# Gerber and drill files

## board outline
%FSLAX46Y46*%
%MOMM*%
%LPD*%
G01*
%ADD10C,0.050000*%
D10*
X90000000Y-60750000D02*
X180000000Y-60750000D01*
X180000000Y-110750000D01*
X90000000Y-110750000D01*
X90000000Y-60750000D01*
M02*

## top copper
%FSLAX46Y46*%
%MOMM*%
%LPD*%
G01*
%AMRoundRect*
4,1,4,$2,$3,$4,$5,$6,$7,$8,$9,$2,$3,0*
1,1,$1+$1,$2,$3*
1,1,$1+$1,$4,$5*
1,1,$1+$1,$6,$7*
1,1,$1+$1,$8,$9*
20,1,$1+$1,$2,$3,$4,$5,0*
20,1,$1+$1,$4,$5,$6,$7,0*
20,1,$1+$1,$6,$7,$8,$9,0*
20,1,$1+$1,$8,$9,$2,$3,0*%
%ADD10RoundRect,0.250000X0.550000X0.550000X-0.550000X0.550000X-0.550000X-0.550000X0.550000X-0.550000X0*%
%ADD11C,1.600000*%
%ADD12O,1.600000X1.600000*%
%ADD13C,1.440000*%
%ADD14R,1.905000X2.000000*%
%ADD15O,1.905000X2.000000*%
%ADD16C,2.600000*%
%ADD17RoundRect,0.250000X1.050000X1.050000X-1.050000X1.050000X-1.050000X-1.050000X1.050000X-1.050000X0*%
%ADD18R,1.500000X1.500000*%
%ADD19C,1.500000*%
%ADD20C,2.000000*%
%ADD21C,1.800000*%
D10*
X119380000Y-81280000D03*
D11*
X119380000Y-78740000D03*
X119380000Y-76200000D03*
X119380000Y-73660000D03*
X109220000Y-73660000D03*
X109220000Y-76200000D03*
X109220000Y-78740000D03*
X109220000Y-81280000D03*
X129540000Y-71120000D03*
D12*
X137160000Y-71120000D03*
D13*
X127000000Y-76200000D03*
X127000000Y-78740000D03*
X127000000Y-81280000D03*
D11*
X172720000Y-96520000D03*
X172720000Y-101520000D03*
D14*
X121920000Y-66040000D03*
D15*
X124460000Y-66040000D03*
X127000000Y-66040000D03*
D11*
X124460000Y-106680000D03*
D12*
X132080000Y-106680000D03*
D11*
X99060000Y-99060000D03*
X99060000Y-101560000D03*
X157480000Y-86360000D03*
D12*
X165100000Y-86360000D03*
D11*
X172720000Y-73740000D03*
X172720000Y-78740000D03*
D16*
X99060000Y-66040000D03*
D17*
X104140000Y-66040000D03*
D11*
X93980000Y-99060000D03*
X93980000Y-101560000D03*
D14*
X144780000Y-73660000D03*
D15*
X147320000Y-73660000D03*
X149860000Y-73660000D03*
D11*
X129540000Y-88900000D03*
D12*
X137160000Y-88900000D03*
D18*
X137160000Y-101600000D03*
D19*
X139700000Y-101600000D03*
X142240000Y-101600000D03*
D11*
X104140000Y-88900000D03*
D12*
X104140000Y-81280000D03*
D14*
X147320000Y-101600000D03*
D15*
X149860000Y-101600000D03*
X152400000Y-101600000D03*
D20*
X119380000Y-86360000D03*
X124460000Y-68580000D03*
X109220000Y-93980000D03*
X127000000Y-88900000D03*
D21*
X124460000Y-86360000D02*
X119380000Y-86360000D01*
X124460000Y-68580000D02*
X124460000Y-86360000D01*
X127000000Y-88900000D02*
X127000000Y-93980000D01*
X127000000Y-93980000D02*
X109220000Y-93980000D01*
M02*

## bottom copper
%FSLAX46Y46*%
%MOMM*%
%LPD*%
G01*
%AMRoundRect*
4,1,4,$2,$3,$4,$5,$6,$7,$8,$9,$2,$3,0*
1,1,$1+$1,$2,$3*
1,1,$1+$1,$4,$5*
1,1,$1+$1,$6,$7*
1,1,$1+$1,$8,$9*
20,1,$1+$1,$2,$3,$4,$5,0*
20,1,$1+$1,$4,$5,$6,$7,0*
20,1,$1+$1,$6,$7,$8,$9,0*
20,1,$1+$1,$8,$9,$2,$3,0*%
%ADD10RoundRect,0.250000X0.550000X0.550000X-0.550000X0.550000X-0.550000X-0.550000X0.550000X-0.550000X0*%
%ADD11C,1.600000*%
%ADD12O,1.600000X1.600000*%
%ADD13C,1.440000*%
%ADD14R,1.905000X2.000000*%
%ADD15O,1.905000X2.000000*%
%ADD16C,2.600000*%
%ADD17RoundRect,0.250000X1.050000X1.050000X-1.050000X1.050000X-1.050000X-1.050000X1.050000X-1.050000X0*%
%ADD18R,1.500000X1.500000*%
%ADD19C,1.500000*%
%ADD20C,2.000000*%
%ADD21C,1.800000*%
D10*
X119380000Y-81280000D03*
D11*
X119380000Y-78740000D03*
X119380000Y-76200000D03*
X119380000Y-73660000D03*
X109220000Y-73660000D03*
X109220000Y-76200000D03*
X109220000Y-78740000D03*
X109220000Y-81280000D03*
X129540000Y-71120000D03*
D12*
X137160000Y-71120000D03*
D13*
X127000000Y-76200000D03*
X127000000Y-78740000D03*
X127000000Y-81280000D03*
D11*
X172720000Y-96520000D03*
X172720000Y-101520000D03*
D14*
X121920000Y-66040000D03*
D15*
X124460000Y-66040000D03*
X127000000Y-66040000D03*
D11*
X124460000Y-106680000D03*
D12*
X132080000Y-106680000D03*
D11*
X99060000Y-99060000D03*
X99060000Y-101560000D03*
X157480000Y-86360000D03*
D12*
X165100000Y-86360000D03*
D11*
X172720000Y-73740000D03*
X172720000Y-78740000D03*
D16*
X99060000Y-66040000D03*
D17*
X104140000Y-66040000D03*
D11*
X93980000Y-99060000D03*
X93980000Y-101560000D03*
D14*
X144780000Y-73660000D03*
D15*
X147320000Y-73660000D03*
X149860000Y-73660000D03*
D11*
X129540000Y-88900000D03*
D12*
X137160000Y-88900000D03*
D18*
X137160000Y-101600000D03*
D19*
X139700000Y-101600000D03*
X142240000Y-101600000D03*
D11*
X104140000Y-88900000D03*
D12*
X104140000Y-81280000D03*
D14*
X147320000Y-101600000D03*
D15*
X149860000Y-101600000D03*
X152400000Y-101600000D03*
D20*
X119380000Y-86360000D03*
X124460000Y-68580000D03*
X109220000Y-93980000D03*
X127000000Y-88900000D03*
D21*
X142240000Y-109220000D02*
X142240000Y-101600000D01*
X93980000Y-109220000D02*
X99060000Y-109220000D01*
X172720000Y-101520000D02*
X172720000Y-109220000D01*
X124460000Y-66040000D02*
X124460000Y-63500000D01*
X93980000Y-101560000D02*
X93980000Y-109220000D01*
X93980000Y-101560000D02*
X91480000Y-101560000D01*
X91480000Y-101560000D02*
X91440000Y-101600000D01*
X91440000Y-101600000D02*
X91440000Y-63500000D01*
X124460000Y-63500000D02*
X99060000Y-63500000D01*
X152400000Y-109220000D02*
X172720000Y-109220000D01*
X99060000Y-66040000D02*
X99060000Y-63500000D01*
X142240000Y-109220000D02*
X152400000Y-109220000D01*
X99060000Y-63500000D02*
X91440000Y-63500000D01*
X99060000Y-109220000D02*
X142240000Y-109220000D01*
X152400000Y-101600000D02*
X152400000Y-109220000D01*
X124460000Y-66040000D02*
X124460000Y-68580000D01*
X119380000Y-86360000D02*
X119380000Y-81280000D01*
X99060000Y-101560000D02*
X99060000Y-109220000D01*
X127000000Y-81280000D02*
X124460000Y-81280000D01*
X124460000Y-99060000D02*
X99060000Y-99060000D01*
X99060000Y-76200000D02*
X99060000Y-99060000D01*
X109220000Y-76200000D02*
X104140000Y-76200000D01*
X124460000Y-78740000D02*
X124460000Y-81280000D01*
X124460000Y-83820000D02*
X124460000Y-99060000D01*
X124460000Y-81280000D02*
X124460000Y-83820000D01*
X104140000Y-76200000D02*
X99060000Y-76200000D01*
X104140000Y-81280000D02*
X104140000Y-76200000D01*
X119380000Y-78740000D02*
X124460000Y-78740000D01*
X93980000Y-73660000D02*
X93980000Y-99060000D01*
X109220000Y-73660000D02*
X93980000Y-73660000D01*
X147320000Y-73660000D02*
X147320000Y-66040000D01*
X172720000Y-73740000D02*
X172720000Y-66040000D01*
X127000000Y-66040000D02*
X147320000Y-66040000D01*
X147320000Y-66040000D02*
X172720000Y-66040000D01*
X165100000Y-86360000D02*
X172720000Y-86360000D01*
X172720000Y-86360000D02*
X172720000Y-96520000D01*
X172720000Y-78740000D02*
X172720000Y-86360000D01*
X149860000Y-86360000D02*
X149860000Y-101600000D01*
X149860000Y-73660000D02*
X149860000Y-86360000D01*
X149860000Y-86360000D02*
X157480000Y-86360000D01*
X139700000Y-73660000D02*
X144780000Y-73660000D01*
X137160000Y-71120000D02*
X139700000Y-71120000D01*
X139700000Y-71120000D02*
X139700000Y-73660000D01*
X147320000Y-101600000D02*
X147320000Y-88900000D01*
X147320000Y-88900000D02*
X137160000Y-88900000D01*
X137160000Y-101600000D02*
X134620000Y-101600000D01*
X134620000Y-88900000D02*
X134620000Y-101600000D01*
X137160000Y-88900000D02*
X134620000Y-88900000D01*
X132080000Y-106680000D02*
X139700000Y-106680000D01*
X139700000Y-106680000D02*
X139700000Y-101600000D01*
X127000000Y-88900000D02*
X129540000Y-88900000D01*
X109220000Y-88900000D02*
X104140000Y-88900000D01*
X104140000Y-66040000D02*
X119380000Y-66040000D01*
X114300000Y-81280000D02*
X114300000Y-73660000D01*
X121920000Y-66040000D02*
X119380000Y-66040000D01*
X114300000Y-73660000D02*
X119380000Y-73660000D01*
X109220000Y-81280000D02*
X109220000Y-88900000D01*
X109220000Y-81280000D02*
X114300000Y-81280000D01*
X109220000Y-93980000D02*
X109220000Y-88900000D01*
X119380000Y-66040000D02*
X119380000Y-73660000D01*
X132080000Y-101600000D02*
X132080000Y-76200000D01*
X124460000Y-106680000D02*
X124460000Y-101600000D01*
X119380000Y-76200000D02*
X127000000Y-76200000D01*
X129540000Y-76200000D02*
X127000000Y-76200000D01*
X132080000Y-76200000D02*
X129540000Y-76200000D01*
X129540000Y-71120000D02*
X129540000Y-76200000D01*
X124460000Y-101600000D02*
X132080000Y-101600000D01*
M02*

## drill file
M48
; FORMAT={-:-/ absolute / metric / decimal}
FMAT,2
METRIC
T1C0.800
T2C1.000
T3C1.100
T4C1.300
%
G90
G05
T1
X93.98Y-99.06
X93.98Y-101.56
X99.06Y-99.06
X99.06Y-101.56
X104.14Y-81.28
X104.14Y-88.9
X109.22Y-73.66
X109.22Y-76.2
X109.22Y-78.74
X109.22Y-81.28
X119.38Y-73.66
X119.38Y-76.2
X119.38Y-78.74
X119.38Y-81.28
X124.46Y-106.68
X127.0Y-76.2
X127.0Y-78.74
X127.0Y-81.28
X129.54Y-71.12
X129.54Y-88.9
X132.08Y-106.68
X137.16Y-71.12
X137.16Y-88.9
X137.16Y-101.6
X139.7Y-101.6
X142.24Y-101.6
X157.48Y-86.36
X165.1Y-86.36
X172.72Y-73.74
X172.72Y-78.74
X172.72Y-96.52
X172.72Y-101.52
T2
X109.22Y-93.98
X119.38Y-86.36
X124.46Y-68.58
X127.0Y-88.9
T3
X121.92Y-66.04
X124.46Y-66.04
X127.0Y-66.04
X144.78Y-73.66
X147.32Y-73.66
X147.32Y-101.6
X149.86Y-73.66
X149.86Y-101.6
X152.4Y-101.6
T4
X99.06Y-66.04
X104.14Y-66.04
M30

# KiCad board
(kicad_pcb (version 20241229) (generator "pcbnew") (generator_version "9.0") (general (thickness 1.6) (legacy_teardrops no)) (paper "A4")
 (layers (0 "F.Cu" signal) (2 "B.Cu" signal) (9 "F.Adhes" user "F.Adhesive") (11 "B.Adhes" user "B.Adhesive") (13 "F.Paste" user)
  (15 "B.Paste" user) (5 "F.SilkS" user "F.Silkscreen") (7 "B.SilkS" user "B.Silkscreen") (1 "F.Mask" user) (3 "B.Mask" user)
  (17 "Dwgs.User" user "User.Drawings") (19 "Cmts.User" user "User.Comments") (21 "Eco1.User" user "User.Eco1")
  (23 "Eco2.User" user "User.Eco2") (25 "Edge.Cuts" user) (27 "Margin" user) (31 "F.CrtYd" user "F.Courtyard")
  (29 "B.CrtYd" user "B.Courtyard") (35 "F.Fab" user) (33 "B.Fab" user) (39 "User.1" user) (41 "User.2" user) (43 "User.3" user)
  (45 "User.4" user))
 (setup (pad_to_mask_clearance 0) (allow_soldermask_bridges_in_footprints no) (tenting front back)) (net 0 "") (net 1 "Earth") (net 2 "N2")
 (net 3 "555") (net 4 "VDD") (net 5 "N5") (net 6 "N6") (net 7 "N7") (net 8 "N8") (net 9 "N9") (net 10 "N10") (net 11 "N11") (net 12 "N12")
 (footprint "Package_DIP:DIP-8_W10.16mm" (layer "F.Cu") (at 119.38 81.28 180)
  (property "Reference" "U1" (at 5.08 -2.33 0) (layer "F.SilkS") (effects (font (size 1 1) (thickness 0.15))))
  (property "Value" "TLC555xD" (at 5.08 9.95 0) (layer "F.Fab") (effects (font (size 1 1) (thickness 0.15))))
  (pad "1" thru_hole roundrect (at 0 0 180) (size 1.6 1.6) (drill 0.8) (layers "*.Cu" "*.Mask") (remove_unused_layers no)
   (roundrect_rratio 0.15625) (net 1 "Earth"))
  (pad "2" thru_hole circle (at 0 2.54 180) (size 1.6 1.6) (drill 0.8) (layers "*.Cu" "*.Mask") (remove_unused_layers no) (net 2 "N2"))
  (pad "3" thru_hole circle (at 0 5.08 180) (size 1.6 1.6) (drill 0.8) (layers "*.Cu" "*.Mask") (remove_unused_layers no) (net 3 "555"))
  (pad "4" thru_hole circle (at 0 7.62 180) (size 1.6 1.6) (drill 0.8) (layers "*.Cu" "*.Mask") (remove_unused_layers no) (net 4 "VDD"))
  (pad "5" thru_hole circle (at 10.16 7.62 180) (size 1.6 1.6) (drill 0.8) (layers "*.Cu" "*.Mask") (remove_unused_layers no) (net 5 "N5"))
  (pad "6" thru_hole circle (at 10.16 5.08 180) (size 1.6 1.6) (drill 0.8) (layers "*.Cu" "*.Mask") (remove_unused_layers no) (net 2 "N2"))
  (pad "7" thru_hole circle (at 10.16 2.54 180) (size 1.6 1.6) (drill 0.8) (layers "*.Cu" "*.Mask") (remove_unused_layers no) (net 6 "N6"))
  (pad "8" thru_hole circle (at 10.16 0 180) (size 1.6 1.6) (drill 0.8) (layers "*.Cu" "*.Mask") (remove_unused_layers no) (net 4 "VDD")))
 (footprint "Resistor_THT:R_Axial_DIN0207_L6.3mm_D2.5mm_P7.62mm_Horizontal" (layer "F.Cu") (at 129.54 71.12)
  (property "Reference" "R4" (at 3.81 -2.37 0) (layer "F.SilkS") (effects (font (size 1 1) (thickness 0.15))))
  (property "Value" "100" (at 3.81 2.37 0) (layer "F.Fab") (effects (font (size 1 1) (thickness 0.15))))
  (pad "1" thru_hole circle (at 0 0) (size 1.6 1.6) (drill 0.8) (layers "*.Cu" "*.Mask") (remove_unused_layers no) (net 3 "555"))
  (pad "2" thru_hole oval (at 7.62 0) (size 1.6 1.6) (drill 0.8) (layers "*.Cu" "*.Mask") (remove_unused_layers no) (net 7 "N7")))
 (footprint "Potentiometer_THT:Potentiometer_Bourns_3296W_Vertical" (layer "F.Cu") (at 127 76.2 90)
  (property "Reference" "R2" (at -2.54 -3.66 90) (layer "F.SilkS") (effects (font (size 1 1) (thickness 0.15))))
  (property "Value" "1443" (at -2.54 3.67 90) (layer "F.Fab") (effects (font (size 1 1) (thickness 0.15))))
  (pad "1" thru_hole circle (at 0 0 90) (size 1.44 1.44) (drill 0.8) (layers "*.Cu" "*.Mask") (remove_unused_layers no) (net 3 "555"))
  (pad "2" thru_hole circle (at -2.54 0 90) (size 1.44 1.44) (drill 0.8) (layers "*.Cu" "*.Mask") (remove_unused_layers no))
  (pad "3" thru_hole circle (at -5.08 0 90) (size 1.44 1.44) (drill 0.8) (layers "*.Cu" "*.Mask") (remove_unused_layers no) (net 2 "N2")))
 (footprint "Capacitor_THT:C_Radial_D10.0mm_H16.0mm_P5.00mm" (layer "F.Cu") (at 172.72 96.52 -90)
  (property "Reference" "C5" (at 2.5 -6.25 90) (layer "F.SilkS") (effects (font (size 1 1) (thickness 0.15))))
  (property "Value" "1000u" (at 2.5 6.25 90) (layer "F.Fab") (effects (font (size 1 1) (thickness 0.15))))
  (pad "1" thru_hole circle (at 0 0 270) (size 1.6 1.6) (drill 0.8) (layers "*.Cu" "*.Mask") (remove_unused_layers no) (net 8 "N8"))
  (pad "2" thru_hole circle (at 5 0 270) (size 1.6 1.6) (drill 0.8) (layers "*.Cu" "*.Mask") (remove_unused_layers no) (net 1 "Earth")))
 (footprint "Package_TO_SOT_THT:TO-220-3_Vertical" (layer "F.Cu") (at 121.92 66.04)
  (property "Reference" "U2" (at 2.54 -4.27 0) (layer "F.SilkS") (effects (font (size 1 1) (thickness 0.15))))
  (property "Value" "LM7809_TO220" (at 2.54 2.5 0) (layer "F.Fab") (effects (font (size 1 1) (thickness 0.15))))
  (pad "1" thru_hole rect (at 0 0) (size 1.905 2) (drill 1.1) (layers "*.Cu" "*.Mask") (remove_unused_layers no) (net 4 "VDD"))
  (pad "2" thru_hole oval (at 2.54 0) (size 1.905 2) (drill 1.1) (layers "*.Cu" "*.Mask") (remove_unused_layers no) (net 1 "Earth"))
  (pad "3" thru_hole oval (at 5.08 0) (size 1.905 2) (drill 1.1) (layers "*.Cu" "*.Mask") (remove_unused_layers no) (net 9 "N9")))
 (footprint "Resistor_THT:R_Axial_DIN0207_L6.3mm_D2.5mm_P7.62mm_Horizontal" (layer "F.Cu") (at 124.46 106.68)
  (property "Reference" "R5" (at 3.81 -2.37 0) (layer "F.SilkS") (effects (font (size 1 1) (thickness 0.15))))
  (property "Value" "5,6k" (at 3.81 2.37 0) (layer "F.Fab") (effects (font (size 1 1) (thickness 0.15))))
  (pad "1" thru_hole circle (at 0 0) (size 1.6 1.6) (drill 0.8) (layers "*.Cu" "*.Mask") (remove_unused_layers no) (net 3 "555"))
  (pad "2" thru_hole oval (at 7.62 0) (size 1.6 1.6) (drill 0.8) (layers "*.Cu" "*.Mask") (remove_unused_layers no) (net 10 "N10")))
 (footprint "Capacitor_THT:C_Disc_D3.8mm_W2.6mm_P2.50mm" (layer "F.Cu") (at 99.06 99.06 -90)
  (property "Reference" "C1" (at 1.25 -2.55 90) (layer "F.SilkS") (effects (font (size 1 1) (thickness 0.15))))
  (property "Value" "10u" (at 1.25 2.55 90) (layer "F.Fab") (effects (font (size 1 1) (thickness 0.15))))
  (pad "1" thru_hole circle (at 0 0 270) (size 1.6 1.6) (drill 0.8) (layers "*.Cu" "*.Mask") (remove_unused_layers no) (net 2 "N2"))
  (pad "2" thru_hole circle (at 2.5 0 270) (size 1.6 1.6) (drill 0.8) (layers "*.Cu" "*.Mask") (remove_unused_layers no) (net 1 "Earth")))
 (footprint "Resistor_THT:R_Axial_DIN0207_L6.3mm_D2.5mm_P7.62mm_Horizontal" (layer "F.Cu") (at 157.48 86.36)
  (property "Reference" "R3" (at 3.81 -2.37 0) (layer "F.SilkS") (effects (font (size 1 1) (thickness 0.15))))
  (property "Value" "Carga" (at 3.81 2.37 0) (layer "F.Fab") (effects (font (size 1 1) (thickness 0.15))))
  (pad "1" thru_hole circle (at 0 0) (size 1.6 1.6) (drill 0.8) (layers "*.Cu" "*.Mask") (remove_unused_layers no) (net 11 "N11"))
  (pad "2" thru_hole oval (at 7.62 0) (size 1.6 1.6) (drill 0.8) (layers "*.Cu" "*.Mask") (remove_unused_layers no) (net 8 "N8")))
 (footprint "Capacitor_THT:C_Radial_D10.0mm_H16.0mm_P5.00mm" (layer "F.Cu") (at 172.72 73.74 -90)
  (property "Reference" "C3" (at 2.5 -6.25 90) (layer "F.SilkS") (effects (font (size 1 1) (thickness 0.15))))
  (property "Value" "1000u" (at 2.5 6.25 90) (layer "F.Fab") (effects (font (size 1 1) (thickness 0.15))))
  (pad "1" thru_hole circle (at 0 0 270) (size 1.6 1.6) (drill 0.8) (layers "*.Cu" "*.Mask") (remove_unused_layers no) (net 9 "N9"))
  (pad "2" thru_hole circle (at 5 0 270) (size 1.6 1.6) (drill 0.8) (layers "*.Cu" "*.Mask") (remove_unused_layers no) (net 8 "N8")))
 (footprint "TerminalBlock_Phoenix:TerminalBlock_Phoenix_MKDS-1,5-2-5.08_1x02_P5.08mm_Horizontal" (layer "F.Cu") (at 104.14 66.04 180)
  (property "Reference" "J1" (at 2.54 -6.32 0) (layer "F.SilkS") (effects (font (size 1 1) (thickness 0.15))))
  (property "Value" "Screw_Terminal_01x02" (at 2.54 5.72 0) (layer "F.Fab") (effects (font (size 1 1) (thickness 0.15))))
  (pad "1" thru_hole circle (at 5.08 0 180) (size 2.6 2.6) (drill 1.3) (layers "*.Cu" "*.Mask") (remove_unused_layers no) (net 1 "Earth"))
  (pad "2" thru_hole roundrect (at 0 0 180) (size 2.6 2.6) (drill 1.3) (layers "*.Cu" "*.Mask") (remove_unused_layers no)
   (roundrect_rratio 0.096154) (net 4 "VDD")))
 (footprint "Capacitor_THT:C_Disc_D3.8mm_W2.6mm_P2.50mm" (layer "F.Cu") (at 93.98 99.06 -90)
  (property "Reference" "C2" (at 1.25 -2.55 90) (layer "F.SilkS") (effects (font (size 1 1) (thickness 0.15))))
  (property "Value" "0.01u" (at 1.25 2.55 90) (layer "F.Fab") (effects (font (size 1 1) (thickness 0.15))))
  (pad "1" thru_hole circle (at 0 0 270) (size 1.6 1.6) (drill 0.8) (layers "*.Cu" "*.Mask") (remove_unused_layers no) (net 5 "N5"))
  (pad "2" thru_hole circle (at 2.5 0 270) (size 1.6 1.6) (drill 0.8) (layers "*.Cu" "*.Mask") (remove_unused_layers no) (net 1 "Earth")))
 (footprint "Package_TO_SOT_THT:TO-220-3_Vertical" (layer "F.Cu") (at 144.78 73.66)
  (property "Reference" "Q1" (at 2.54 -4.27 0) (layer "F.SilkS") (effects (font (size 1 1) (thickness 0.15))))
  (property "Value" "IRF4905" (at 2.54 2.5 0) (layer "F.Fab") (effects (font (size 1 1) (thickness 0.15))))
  (pad "1" thru_hole rect (at 0 0) (size 1.905 2) (drill 1.1) (layers "*.Cu" "*.Mask") (remove_unused_layers no) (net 7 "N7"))
  (pad "2" thru_hole oval (at 2.54 0) (size 1.905 2) (drill 1.1) (layers "*.Cu" "*.Mask") (remove_unused_layers no) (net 9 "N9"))
  (pad "3" thru_hole oval (at 5.08 0) (size 1.905 2) (drill 1.1) (layers "*.Cu" "*.Mask") (remove_unused_layers no) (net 11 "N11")))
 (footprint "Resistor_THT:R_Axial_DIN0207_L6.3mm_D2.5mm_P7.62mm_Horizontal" (layer "F.Cu") (at 129.54 88.9)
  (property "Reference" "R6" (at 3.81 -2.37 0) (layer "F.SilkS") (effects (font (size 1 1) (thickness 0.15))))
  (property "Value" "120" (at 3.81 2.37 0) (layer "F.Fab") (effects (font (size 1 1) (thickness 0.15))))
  (pad "1" thru_hole circle (at 0 0) (size 1.6 1.6) (drill 0.8) (layers "*.Cu" "*.Mask") (remove_unused_layers no) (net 4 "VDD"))
  (pad "2" thru_hole oval (at 7.62 0) (size 1.6 1.6) (drill 0.8) (layers "*.Cu" "*.Mask") (remove_unused_layers no) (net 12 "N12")))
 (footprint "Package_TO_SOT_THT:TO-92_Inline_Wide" (layer "F.Cu") (at 137.16 101.6)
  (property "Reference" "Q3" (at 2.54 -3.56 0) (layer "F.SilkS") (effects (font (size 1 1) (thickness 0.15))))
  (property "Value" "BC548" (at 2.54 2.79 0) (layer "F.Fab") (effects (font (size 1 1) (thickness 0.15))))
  (pad "1" thru_hole rect (at 0 0) (size 1.5 1.5) (drill 0.8) (layers "*.Cu" "*.Mask") (remove_unused_layers no) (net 12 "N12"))
  (pad "2" thru_hole circle (at 2.54 0) (size 1.5 1.5) (drill 0.8) (layers "*.Cu" "*.Mask") (remove_unused_layers no) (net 10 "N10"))
  (pad "3" thru_hole circle (at 5.08 0) (size 1.5 1.5) (drill 0.8) (layers "*.Cu" "*.Mask") (remove_unused_layers no) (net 1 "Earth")))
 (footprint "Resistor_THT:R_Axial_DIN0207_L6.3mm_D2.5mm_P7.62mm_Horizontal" (layer "F.Cu") (at 104.14 88.9 90)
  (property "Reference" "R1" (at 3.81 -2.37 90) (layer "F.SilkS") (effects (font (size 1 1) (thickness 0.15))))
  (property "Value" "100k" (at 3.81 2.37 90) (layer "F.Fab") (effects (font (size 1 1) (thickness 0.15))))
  (pad "1" thru_hole circle (at 0 0 90) (size 1.6 1.6) (drill 0.8) (layers "*.Cu" "*.Mask") (remove_unused_layers no) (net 4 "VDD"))
  (pad "2" thru_hole oval (at 7.62 0 90) (size 1.6 1.6) (drill 0.8) (layers "*.Cu" "*.Mask") (remove_unused_layers no) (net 2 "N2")))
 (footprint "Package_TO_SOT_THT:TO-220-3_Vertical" (layer "F.Cu") (at 147.32 101.6)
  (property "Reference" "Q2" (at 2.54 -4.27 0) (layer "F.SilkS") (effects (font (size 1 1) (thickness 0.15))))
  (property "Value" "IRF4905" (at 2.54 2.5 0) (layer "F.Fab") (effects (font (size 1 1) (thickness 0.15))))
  (pad "1" thru_hole rect (at 0 0) (size 1.905 2) (drill 1.1) (layers "*.Cu" "*.Mask") (remove_unused_layers no) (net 12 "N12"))
  (pad "2" thru_hole oval (at 2.54 0) (size 1.905 2) (drill 1.1) (layers "*.Cu" "*.Mask") (remove_unused_layers no) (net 11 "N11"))
  (pad "3" thru_hole oval (at 5.08 0) (size 1.905 2) (drill 1.1) (layers "*.Cu" "*.Mask") (remove_unused_layers no) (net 1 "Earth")))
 (gr_rect (start 90 60.75) (end 180 110.75) (stroke (width 0.05) (type solid)) (fill no) (layer "Edge.Cuts"))
 (segment (start 124.46 86.36) (end 119.38 86.36) (width 1.8) (layer "F.Cu") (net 1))
 (segment (start 124.46 68.58) (end 124.46 86.36) (width 1.8) (layer "F.Cu") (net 1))
 (via (at 119.38 86.36) (size 2) (drill 1) (layers "F.Cu" "B.Cu") (free yes) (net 1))
 (via (at 124.46 68.58) (size 2) (drill 1) (layers "F.Cu" "B.Cu") (free yes) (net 1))
 (segment (start 142.24 109.22) (end 142.24 101.6) (width 1.8) (layer "B.Cu") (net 1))
 (segment (start 93.98 109.22) (end 99.06 109.22) (width 1.8) (layer "B.Cu") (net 1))
 (segment (start 172.72 101.52) (end 172.72 109.22) (width 1.8) (layer "B.Cu") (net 1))
 (segment (start 124.46 66.04) (end 124.46 63.5) (width 1.8) (layer "B.Cu") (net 1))
 (segment (start 93.98 101.56) (end 93.98 109.22) (width 1.8) (layer "B.Cu") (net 1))
 (segment (start 93.98 101.56) (end 91.48 101.56) (width 1.8) (layer "B.Cu") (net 1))
 (segment (start 91.48 101.56) (end 91.44 101.6) (width 1.8) (layer "B.Cu") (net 1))
 (segment (start 91.44 101.6) (end 91.44 63.5) (width 1.8) (layer "B.Cu") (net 1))
 (segment (start 124.46 63.5) (end 99.06 63.5) (width 1.8) (layer "B.Cu") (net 1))
 (segment (start 152.4 109.22) (end 172.72 109.22) (width 1.8) (layer "B.Cu") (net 1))
 (segment (start 99.06 66.04) (end 99.06 63.5) (width 1.8) (layer "B.Cu") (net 1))
 (segment (start 142.24 109.22) (end 152.4 109.22) (width 1.8) (layer "B.Cu") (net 1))
 (segment (start 99.06 63.5) (end 91.44 63.5) (width 1.8) (layer "B.Cu") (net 1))
 (segment (start 99.06 109.22) (end 142.24 109.22) (width 1.8) (layer "B.Cu") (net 1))
 (segment (start 152.4 101.6) (end 152.4 109.22) (width 1.8) (layer "B.Cu") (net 1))
 (segment (start 124.46 66.04) (end 124.46 68.58) (width 1.8) (layer "B.Cu") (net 1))
 (segment (start 119.38 86.36) (end 119.38 81.28) (width 1.8) (layer "B.Cu") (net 1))
 (segment (start 99.06 101.56) (end 99.06 109.22) (width 1.8) (layer "B.Cu") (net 1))
 (segment (start 127 81.28) (end 124.46 81.28) (width 1.8) (layer "B.Cu") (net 2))
 (segment (start 124.46 99.06) (end 99.06 99.06) (width 1.8) (layer "B.Cu") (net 2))
 (segment (start 99.06 76.2) (end 99.06 99.06) (width 1.8) (layer "B.Cu") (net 2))
 (segment (start 109.22 76.2) (end 104.14 76.2) (width 1.8) (layer "B.Cu") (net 2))
 (segment (start 124.46 78.74) (end 124.46 81.28) (width 1.8) (layer "B.Cu") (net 2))
 (segment (start 124.46 83.82) (end 124.46 99.06) (width 1.8) (layer "B.Cu") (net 2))
 (segment (start 124.46 81.28) (end 124.46 83.82) (width 1.8) (layer "B.Cu") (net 2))
 (segment (start 104.14 76.2) (end 99.06 76.2) (width 1.8) (layer "B.Cu") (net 2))
 (segment (start 104.14 81.28) (end 104.14 76.2) (width 1.8) (layer "B.Cu") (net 2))
 (segment (start 119.38 78.74) (end 124.46 78.74) (width 1.8) (layer "B.Cu") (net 2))
 (segment (start 93.98 73.66) (end 93.98 99.06) (width 1.8) (layer "B.Cu") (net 5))
 (segment (start 109.22 73.66) (end 93.98 73.66) (width 1.8) (layer "B.Cu") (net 5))
 (segment (start 147.32 73.66) (end 147.32 66.04) (width 1.8) (layer "B.Cu") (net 9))
 (segment (start 172.72 73.74) (end 172.72 66.04) (width 1.8) (layer "B.Cu") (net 9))
 (segment (start 127 66.04) (end 147.32 66.04) (width 1.8) (layer "B.Cu") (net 9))
 (segment (start 147.32 66.04) (end 172.72 66.04) (width 1.8) (layer "B.Cu") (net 9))
 (segment (start 165.1 86.36) (end 172.72 86.36) (width 1.8) (layer "B.Cu") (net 8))
 (segment (start 172.72 86.36) (end 172.72 96.52) (width 1.8) (layer "B.Cu") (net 8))
 (segment (start 172.72 78.74) (end 172.72 86.36) (width 1.8) (layer "B.Cu") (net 8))
 (segment (start 149.86 86.36) (end 149.86 101.6) (width 1.8) (layer "B.Cu") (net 11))
 (segment (start 149.86 73.66) (end 149.86 86.36) (width 1.8) (layer "B.Cu") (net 11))
 (segment (start 149.86 86.36) (end 157.48 86.36) (width 1.8) (layer "B.Cu") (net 11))
 (segment (start 139.7 73.66) (end 144.78 73.66) (width 1.8) (layer "B.Cu") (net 7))
 (segment (start 137.16 71.12) (end 139.7 71.12) (width 1.8) (layer "B.Cu") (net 7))
 (segment (start 139.7 71.12) (end 139.7 73.66) (width 1.8) (layer "B.Cu") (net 7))
 (segment (start 147.32 101.6) (end 147.32 88.9) (width 1.8) (layer "B.Cu") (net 12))
 (segment (start 147.32 88.9) (end 137.16 88.9) (width 1.8) (layer "B.Cu") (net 12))
 (segment (start 137.16 101.6) (end 134.62 101.6) (width 1.8) (layer "B.Cu") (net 12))
 (segment (start 134.62 88.9) (end 134.62 101.6) (width 1.8) (layer "B.Cu") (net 12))
 (segment (start 137.16 88.9) (end 134.62 88.9) (width 1.8) (layer "B.Cu") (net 12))
 (segment (start 132.08 106.68) (end 139.7 106.68) (width 1.8) (layer "B.Cu") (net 10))
 (segment (start 139.7 106.68) (end 139.7 101.6) (width 1.8) (layer "B.Cu") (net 10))
 (segment (start 127 88.9) (end 127 93.98) (width 1.8) (layer "F.Cu") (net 4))
 (segment (start 127 93.98) (end 109.22 93.98) (width 1.8) (layer "F.Cu") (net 4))
 (via (at 109.22 93.98) (size 2) (drill 1) (layers "F.Cu" "B.Cu") (free yes) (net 4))
 (via (at 127 88.9) (size 2) (drill 1) (layers "F.Cu" "B.Cu") (free yes) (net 4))
 (segment (start 127 88.9) (end 129.54 88.9) (width 1.8) (layer "B.Cu") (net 4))
 (segment (start 109.22 88.9) (end 104.14 88.9) (width 1.8) (layer "B.Cu") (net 4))
 (segment (start 104.14 66.04) (end 119.38 66.04) (width 1.8) (layer "B.Cu") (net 4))
 (segment (start 114.3 81.28) (end 114.3 73.66) (width 1.8) (layer "B.Cu") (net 4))
 (segment (start 121.92 66.04) (end 119.38 66.04) (width 1.8) (layer "B.Cu") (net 4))
 (segment (start 114.3 73.66) (end 119.38 73.66) (width 1.8) (layer "B.Cu") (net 4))
 (segment (start 109.22 81.28) (end 109.22 88.9) (width 1.8) (layer "B.Cu") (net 4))
 (segment (start 109.22 81.28) (end 114.3 81.28) (width 1.8) (layer "B.Cu") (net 4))
 (segment (start 109.22 93.98) (end 109.22 88.9) (width 1.8) (layer "B.Cu") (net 4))
 (segment (start 119.38 66.04) (end 119.38 73.66) (width 1.8) (layer "B.Cu") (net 4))
 (segment (start 132.08 101.6) (end 132.08 76.2) (width 1.8) (layer "B.Cu") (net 3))
 (segment (start 124.46 106.68) (end 124.46 101.6) (width 1.8) (layer "B.Cu") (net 3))
 (segment (start 119.38 76.2) (end 127 76.2) (width 1.8) (layer "B.Cu") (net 3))
 (segment (start 129.54 76.2) (end 127 76.2) (width 1.8) (layer "B.Cu") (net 3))
 (segment (start 132.08 76.2) (end 129.54 76.2) (width 1.8) (layer "B.Cu") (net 3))
 (segment (start 129.54 71.12) (end 129.54 76.2) (width 1.8) (layer "B.Cu") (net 3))
 (segment (start 124.46 101.6) (end 132.08 101.6) (width 1.8) (layer "B.Cu") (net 3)))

